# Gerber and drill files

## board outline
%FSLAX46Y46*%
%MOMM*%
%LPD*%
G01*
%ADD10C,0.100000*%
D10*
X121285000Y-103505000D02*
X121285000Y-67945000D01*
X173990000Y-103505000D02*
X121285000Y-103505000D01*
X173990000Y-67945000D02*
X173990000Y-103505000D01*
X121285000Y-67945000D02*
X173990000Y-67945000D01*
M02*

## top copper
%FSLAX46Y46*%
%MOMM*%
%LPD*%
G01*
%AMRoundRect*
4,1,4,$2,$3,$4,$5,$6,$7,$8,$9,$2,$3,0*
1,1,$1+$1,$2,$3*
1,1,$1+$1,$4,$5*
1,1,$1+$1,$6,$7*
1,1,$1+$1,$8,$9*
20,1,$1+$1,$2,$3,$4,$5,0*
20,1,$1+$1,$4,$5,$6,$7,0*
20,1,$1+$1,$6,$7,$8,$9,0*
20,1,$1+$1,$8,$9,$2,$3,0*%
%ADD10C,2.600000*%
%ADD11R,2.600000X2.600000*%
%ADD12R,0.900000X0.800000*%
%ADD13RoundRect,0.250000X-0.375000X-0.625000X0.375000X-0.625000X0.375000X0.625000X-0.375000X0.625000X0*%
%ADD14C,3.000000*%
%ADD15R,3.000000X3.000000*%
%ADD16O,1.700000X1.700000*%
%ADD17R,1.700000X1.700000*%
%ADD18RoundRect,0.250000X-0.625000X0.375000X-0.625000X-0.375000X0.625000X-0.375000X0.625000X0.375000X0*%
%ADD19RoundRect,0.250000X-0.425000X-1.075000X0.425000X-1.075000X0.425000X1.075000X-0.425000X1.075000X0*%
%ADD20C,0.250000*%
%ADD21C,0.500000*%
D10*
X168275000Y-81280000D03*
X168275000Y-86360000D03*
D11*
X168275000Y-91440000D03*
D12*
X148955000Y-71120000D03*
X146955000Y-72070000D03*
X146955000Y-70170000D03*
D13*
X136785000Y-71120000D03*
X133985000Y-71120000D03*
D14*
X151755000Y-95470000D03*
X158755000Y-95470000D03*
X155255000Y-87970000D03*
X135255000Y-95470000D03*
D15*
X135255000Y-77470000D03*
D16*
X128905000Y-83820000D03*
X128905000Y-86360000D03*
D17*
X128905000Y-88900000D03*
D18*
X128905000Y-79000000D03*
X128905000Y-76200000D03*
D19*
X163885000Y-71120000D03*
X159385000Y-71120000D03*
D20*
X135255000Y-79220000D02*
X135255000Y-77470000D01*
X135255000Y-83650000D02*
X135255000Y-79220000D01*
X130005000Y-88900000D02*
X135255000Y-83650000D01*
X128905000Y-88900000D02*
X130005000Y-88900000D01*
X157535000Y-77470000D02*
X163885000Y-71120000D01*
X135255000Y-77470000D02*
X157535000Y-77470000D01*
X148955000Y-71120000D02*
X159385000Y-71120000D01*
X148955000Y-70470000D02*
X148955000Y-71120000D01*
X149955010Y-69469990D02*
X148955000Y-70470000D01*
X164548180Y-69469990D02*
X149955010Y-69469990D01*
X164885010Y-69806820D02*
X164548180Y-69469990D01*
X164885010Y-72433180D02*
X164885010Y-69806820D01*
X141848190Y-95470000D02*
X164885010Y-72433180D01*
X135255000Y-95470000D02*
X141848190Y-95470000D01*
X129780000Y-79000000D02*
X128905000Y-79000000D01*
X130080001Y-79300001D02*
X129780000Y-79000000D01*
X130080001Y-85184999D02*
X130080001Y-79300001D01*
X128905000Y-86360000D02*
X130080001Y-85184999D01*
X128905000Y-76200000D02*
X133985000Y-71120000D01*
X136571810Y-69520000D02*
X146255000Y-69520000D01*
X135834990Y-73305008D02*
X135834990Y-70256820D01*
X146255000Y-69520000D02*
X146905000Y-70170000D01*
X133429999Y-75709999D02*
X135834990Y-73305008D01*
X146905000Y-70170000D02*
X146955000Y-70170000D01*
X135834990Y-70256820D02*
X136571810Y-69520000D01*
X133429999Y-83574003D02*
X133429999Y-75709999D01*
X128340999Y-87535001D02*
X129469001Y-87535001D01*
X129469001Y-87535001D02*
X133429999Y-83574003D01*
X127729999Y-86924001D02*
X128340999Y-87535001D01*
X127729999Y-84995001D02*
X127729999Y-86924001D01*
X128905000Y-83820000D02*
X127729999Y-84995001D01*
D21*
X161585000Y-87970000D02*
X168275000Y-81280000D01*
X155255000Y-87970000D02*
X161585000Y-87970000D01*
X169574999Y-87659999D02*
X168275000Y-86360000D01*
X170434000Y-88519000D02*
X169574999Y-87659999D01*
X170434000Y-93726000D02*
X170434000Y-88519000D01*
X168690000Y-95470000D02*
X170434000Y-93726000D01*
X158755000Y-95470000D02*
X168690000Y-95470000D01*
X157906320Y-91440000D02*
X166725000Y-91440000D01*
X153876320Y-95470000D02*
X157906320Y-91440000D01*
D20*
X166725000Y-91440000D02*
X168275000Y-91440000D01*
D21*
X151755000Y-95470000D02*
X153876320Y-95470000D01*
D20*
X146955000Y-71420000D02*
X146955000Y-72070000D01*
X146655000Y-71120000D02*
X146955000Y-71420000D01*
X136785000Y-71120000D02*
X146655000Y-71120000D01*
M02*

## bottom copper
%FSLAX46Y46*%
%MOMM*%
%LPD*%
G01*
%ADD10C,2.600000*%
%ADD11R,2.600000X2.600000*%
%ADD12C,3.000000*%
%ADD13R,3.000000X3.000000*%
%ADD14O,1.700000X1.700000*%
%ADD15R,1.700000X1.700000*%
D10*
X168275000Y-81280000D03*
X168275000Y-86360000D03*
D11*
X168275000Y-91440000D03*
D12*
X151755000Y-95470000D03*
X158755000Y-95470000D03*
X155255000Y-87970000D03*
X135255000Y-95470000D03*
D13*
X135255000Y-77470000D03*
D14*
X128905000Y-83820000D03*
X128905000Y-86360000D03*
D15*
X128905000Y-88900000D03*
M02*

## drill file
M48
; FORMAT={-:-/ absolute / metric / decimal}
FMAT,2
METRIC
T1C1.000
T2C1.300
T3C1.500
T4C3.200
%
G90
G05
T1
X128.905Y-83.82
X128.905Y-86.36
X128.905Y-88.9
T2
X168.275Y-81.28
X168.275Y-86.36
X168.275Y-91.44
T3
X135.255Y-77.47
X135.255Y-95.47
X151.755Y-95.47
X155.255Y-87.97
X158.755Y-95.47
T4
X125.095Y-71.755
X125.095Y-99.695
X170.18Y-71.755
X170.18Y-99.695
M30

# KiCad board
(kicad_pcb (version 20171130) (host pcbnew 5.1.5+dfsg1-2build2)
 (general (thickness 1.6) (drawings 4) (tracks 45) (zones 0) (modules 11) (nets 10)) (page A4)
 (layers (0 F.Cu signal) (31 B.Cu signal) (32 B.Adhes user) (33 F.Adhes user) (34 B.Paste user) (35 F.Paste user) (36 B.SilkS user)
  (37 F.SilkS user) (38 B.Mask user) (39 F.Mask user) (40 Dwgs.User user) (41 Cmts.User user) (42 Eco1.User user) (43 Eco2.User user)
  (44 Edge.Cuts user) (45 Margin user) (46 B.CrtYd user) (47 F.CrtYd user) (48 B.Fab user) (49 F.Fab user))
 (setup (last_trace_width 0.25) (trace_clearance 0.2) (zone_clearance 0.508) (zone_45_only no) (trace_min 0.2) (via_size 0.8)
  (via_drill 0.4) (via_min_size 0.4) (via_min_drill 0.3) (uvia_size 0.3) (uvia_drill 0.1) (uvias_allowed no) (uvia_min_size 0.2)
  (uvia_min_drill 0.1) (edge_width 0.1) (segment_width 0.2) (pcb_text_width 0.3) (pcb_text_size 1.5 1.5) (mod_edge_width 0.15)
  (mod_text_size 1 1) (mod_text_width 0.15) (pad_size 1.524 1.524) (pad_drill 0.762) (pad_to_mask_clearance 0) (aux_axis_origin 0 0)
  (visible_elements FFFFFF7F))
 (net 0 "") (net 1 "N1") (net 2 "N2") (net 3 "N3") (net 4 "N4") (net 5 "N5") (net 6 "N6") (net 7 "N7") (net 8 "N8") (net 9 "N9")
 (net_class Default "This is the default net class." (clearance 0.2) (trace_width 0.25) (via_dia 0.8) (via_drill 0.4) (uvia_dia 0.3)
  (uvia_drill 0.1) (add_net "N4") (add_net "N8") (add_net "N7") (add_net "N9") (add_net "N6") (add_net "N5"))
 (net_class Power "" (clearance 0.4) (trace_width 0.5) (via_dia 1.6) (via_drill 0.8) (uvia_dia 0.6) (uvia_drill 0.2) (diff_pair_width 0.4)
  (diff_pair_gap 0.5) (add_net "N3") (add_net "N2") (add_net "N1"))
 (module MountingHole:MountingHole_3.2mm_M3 (layer F.Cu) (at 125.095 99.695)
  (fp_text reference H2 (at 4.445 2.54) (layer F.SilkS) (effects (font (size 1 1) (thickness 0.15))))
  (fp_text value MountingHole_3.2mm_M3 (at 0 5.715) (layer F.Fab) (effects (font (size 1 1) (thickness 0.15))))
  (pad 1 np_thru_hole circle (at 0 0) (size 3.2 3.2) (drill 3.2) (layers *.Cu *.Mask)))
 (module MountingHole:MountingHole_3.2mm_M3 (layer F.Cu) (at 170.18 99.695)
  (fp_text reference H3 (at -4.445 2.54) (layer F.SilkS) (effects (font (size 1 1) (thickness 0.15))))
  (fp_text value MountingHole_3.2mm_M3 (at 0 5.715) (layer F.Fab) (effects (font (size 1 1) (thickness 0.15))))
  (pad 1 np_thru_hole circle (at 0 0) (size 3.2 3.2) (drill 3.2) (layers *.Cu *.Mask)))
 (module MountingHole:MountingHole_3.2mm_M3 (layer F.Cu) (at 125.095 71.755)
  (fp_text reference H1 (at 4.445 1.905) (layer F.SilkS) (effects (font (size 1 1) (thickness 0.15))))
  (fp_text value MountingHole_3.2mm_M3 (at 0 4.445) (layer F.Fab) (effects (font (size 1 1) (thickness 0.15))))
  (pad 1 np_thru_hole circle (at 0 0) (size 3.2 3.2) (drill 3.2) (layers *.Cu *.Mask)))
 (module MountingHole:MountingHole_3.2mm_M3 (layer F.Cu) (at 170.18 71.755)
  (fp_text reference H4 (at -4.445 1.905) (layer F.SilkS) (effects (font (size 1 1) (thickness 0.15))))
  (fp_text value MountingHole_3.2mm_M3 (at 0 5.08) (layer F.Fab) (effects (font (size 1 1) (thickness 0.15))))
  (pad 1 np_thru_hole circle (at 0 0) (size 3.2 3.2) (drill 3.2) (layers *.Cu *.Mask)))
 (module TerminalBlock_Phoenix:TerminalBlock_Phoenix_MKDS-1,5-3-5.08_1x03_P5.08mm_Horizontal (layer F.Cu) (at 168.275 91.44 90)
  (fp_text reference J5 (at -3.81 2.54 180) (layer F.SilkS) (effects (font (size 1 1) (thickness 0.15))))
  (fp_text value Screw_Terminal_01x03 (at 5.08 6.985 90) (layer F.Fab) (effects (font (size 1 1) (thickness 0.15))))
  (pad 3 thru_hole circle (at 10.16 0 90) (size 2.6 2.6) (drill 1.3) (layers *.Cu *.Mask) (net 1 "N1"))
  (pad 2 thru_hole circle (at 5.08 0 90) (size 2.6 2.6) (drill 1.3) (layers *.Cu *.Mask) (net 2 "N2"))
  (pad 1 thru_hole rect (at 0 0 90) (size 2.6 2.6) (drill 1.3) (layers *.Cu *.Mask) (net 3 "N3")))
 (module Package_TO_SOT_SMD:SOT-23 (layer F.Cu) (at 147.955 71.12)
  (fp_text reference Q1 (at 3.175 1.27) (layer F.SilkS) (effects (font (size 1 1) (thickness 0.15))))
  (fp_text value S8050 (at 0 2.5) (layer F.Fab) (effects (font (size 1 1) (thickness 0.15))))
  (pad 3 smd rect (at 1 0) (size 0.9 0.8) (layers F.Cu F.Paste F.Mask) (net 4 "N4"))
  (pad 2 smd rect (at -1 0.95) (size 0.9 0.8) (layers F.Cu F.Paste F.Mask) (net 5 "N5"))
  (pad 1 smd rect (at -1 -0.95) (size 0.9 0.8) (layers F.Cu F.Paste F.Mask) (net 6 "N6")))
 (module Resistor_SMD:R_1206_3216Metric (layer F.Cu) (at 135.385 71.12)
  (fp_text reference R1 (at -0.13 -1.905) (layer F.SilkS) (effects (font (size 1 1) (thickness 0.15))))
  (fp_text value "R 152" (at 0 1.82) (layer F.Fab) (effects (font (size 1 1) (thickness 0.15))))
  (pad 2 smd roundrect (at 1.4 0) (size 1.25 1.75) (layers F.Cu F.Paste F.Mask) (roundrect_rratio 0.2) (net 5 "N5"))
  (pad 1 smd roundrect (at -1.4 0) (size 1.25 1.75) (layers F.Cu F.Paste F.Mask) (roundrect_rratio 0.2) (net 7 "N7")))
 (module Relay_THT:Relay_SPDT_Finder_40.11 (layer F.Cu) (at 135.255 77.47)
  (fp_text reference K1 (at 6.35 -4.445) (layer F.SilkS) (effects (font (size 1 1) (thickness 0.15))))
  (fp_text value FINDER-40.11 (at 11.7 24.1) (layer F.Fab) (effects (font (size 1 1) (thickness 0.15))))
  (pad 12 thru_hole circle (at 16.5 18) (size 3 3) (drill 1.5) (layers *.Cu *.Mask) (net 3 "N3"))
  (pad 14 thru_hole circle (at 23.5 18) (size 3 3) (drill 1.5) (layers *.Cu *.Mask) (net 2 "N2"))
  (pad 11 thru_hole circle (at 20 10.5) (size 3 3) (drill 1.5) (layers *.Cu *.Mask) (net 1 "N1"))
  (pad A2 thru_hole circle (at 0 18) (size 3 3) (drill 1.5) (layers *.Cu *.Mask) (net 4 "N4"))
  (pad A1 thru_hole rect (at 0 0) (size 3 3) (drill 1.5) (layers *.Cu *.Mask) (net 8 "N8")))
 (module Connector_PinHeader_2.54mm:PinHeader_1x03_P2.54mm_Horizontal (layer F.Cu) (at 128.905 88.9 180)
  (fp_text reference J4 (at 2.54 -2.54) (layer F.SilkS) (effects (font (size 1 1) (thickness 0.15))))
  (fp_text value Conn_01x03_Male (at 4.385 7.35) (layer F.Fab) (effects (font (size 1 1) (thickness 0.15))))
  (pad 3 thru_hole oval (at 0 5.08 180) (size 1.7 1.7) (drill 1) (layers *.Cu *.Mask) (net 6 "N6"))
  (pad 2 thru_hole oval (at 0 2.54 180) (size 1.7 1.7) (drill 1) (layers *.Cu *.Mask) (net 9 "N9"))
  (pad 1 thru_hole rect (at 0 0 180) (size 1.7 1.7) (drill 1) (layers *.Cu *.Mask) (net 8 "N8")))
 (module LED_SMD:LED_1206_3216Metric (layer F.Cu) (at 128.905 77.6 270)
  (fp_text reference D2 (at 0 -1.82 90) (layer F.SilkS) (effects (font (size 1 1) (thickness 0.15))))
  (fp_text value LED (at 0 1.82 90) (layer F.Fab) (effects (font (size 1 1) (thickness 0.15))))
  (pad 2 smd roundrect (at 1.4 0 270) (size 1.25 1.75) (layers F.Cu F.Paste F.Mask) (roundrect_rratio 0.2) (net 9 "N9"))
  (pad 1 smd roundrect (at -1.4 0 270) (size 1.25 1.75) (layers F.Cu F.Paste F.Mask) (roundrect_rratio 0.2) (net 7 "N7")))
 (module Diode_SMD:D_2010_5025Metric (layer F.Cu) (at 161.635 71.12)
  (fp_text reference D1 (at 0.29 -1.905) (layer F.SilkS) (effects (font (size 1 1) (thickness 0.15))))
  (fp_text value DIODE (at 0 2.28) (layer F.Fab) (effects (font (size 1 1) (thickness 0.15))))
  (pad 2 smd roundrect (at 2.25 0) (size 1.35 2.65) (layers F.Cu F.Paste F.Mask) (roundrect_rratio 0.185185) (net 8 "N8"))
  (pad 1 smd roundrect (at -2.25 0) (size 1.35 2.65) (layers F.Cu F.Paste F.Mask) (roundrect_rratio 0.185185) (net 4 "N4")))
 (gr_line (start 121.285 103.505) (end 121.285 67.945) (layer Edge.Cuts) (width 0.1))
 (gr_line (start 173.99 103.505) (end 121.285 103.505) (layer Edge.Cuts) (width 0.1))
 (gr_line (start 173.99 67.945) (end 173.99 103.505) (layer Edge.Cuts) (width 0.1))
 (gr_line (start 121.285 67.945) (end 173.99 67.945) (layer Edge.Cuts) (width 0.1))
 (segment (start 135.255 79.22) (end 135.255 77.47) (width 0.25) (layer F.Cu) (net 8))
 (segment (start 135.255 83.65) (end 135.255 79.22) (width 0.25) (layer F.Cu) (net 8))
 (segment (start 130.005 88.9) (end 135.255 83.65) (width 0.25) (layer F.Cu) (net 8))
 (segment (start 128.905 88.9) (end 130.005 88.9) (width 0.25) (layer F.Cu) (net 8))
 (segment (start 157.535 77.47) (end 163.885 71.12) (width 0.25) (layer F.Cu) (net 8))
 (segment (start 135.255 77.47) (end 157.535 77.47) (width 0.25) (layer F.Cu) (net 8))
 (segment (start 148.955 71.12) (end 159.385 71.12) (width 0.25) (layer F.Cu) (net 4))
 (segment (start 148.955 70.47) (end 148.955 71.12) (width 0.25) (layer F.Cu) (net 4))
 (segment (start 149.95501 69.46999) (end 148.955 70.47) (width 0.25) (layer F.Cu) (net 4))
 (segment (start 164.54818 69.46999) (end 149.95501 69.46999) (width 0.25) (layer F.Cu) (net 4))
 (segment (start 164.88501 69.80682) (end 164.54818 69.46999) (width 0.25) (layer F.Cu) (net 4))
 (segment (start 164.88501 72.43318) (end 164.88501 69.80682) (width 0.25) (layer F.Cu) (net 4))
 (segment (start 141.84819 95.47) (end 164.88501 72.43318) (width 0.25) (layer F.Cu) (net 4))
 (segment (start 135.255 95.47) (end 141.84819 95.47) (width 0.25) (layer F.Cu) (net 4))
 (segment (start 129.78 79) (end 128.905 79) (width 0.25) (layer F.Cu) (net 9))
 (segment (start 130.080001 79.300001) (end 129.78 79) (width 0.25) (layer F.Cu) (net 9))
 (segment (start 130.080001 85.184999) (end 130.080001 79.300001) (width 0.25) (layer F.Cu) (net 9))
 (segment (start 128.905 86.36) (end 130.080001 85.184999) (width 0.25) (layer F.Cu) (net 9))
 (segment (start 128.905 76.2) (end 133.985 71.12) (width 0.25) (layer F.Cu) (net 7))
 (segment (start 136.57181 69.52) (end 146.255 69.52) (width 0.25) (layer F.Cu) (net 6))
 (segment (start 135.83499 73.305008) (end 135.83499 70.25682) (width 0.25) (layer F.Cu) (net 6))
 (segment (start 146.255 69.52) (end 146.905 70.17) (width 0.25) (layer F.Cu) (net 6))
 (segment (start 133.429999 75.709999) (end 135.83499 73.305008) (width 0.25) (layer F.Cu) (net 6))
 (segment (start 146.905 70.17) (end 146.955 70.17) (width 0.25) (layer F.Cu) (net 6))
 (segment (start 135.83499 70.25682) (end 136.57181 69.52) (width 0.25) (layer F.Cu) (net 6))
 (segment (start 133.429999 83.574003) (end 133.429999 75.709999) (width 0.25) (layer F.Cu) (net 6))
 (segment (start 128.340999 87.535001) (end 129.469001 87.535001) (width 0.25) (layer F.Cu) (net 6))
 (segment (start 129.469001 87.535001) (end 133.429999 83.574003) (width 0.25) (layer F.Cu) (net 6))
 (segment (start 127.729999 86.924001) (end 128.340999 87.535001) (width 0.25) (layer F.Cu) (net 6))
 (segment (start 127.729999 84.995001) (end 127.729999 86.924001) (width 0.25) (layer F.Cu) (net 6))
 (segment (start 128.905 83.82) (end 127.729999 84.995001) (width 0.25) (layer F.Cu) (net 6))
 (segment (start 161.585 87.97) (end 168.275 81.28) (width 0.5) (layer F.Cu) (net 1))
 (segment (start 155.255 87.97) (end 161.585 87.97) (width 0.5) (layer F.Cu) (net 1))
 (segment (start 169.574999 87.659999) (end 168.275 86.36) (width 0.5) (layer F.Cu) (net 2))
 (segment (start 170.434 88.519) (end 169.574999 87.659999) (width 0.5) (layer F.Cu) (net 2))
 (segment (start 170.434 93.726) (end 170.434 88.519) (width 0.5) (layer F.Cu) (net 2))
 (segment (start 168.69 95.47) (end 170.434 93.726) (width 0.5) (layer F.Cu) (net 2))
 (segment (start 158.755 95.47) (end 168.69 95.47) (width 0.5) (layer F.Cu) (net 2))
 (segment (start 157.90632 91.44) (end 166.725 91.44) (width 0.5) (layer F.Cu) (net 3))
 (segment (start 153.87632 95.47) (end 157.90632 91.44) (width 0.5) (layer F.Cu) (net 3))
 (segment (start 166.725 91.44) (end 168.275 91.44) (width 0.25) (layer F.Cu) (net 3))
 (segment (start 151.755 95.47) (end 153.87632 95.47) (width 0.5) (layer F.Cu) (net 3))
 (segment (start 146.955 71.42) (end 146.955 72.07) (width 0.25) (layer F.Cu) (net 5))
 (segment (start 146.655 71.12) (end 146.955 71.42) (width 0.25) (layer F.Cu) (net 5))
 (segment (start 136.785 71.12) (end 146.655 71.12) (width 0.25) (layer F.Cu) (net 5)))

